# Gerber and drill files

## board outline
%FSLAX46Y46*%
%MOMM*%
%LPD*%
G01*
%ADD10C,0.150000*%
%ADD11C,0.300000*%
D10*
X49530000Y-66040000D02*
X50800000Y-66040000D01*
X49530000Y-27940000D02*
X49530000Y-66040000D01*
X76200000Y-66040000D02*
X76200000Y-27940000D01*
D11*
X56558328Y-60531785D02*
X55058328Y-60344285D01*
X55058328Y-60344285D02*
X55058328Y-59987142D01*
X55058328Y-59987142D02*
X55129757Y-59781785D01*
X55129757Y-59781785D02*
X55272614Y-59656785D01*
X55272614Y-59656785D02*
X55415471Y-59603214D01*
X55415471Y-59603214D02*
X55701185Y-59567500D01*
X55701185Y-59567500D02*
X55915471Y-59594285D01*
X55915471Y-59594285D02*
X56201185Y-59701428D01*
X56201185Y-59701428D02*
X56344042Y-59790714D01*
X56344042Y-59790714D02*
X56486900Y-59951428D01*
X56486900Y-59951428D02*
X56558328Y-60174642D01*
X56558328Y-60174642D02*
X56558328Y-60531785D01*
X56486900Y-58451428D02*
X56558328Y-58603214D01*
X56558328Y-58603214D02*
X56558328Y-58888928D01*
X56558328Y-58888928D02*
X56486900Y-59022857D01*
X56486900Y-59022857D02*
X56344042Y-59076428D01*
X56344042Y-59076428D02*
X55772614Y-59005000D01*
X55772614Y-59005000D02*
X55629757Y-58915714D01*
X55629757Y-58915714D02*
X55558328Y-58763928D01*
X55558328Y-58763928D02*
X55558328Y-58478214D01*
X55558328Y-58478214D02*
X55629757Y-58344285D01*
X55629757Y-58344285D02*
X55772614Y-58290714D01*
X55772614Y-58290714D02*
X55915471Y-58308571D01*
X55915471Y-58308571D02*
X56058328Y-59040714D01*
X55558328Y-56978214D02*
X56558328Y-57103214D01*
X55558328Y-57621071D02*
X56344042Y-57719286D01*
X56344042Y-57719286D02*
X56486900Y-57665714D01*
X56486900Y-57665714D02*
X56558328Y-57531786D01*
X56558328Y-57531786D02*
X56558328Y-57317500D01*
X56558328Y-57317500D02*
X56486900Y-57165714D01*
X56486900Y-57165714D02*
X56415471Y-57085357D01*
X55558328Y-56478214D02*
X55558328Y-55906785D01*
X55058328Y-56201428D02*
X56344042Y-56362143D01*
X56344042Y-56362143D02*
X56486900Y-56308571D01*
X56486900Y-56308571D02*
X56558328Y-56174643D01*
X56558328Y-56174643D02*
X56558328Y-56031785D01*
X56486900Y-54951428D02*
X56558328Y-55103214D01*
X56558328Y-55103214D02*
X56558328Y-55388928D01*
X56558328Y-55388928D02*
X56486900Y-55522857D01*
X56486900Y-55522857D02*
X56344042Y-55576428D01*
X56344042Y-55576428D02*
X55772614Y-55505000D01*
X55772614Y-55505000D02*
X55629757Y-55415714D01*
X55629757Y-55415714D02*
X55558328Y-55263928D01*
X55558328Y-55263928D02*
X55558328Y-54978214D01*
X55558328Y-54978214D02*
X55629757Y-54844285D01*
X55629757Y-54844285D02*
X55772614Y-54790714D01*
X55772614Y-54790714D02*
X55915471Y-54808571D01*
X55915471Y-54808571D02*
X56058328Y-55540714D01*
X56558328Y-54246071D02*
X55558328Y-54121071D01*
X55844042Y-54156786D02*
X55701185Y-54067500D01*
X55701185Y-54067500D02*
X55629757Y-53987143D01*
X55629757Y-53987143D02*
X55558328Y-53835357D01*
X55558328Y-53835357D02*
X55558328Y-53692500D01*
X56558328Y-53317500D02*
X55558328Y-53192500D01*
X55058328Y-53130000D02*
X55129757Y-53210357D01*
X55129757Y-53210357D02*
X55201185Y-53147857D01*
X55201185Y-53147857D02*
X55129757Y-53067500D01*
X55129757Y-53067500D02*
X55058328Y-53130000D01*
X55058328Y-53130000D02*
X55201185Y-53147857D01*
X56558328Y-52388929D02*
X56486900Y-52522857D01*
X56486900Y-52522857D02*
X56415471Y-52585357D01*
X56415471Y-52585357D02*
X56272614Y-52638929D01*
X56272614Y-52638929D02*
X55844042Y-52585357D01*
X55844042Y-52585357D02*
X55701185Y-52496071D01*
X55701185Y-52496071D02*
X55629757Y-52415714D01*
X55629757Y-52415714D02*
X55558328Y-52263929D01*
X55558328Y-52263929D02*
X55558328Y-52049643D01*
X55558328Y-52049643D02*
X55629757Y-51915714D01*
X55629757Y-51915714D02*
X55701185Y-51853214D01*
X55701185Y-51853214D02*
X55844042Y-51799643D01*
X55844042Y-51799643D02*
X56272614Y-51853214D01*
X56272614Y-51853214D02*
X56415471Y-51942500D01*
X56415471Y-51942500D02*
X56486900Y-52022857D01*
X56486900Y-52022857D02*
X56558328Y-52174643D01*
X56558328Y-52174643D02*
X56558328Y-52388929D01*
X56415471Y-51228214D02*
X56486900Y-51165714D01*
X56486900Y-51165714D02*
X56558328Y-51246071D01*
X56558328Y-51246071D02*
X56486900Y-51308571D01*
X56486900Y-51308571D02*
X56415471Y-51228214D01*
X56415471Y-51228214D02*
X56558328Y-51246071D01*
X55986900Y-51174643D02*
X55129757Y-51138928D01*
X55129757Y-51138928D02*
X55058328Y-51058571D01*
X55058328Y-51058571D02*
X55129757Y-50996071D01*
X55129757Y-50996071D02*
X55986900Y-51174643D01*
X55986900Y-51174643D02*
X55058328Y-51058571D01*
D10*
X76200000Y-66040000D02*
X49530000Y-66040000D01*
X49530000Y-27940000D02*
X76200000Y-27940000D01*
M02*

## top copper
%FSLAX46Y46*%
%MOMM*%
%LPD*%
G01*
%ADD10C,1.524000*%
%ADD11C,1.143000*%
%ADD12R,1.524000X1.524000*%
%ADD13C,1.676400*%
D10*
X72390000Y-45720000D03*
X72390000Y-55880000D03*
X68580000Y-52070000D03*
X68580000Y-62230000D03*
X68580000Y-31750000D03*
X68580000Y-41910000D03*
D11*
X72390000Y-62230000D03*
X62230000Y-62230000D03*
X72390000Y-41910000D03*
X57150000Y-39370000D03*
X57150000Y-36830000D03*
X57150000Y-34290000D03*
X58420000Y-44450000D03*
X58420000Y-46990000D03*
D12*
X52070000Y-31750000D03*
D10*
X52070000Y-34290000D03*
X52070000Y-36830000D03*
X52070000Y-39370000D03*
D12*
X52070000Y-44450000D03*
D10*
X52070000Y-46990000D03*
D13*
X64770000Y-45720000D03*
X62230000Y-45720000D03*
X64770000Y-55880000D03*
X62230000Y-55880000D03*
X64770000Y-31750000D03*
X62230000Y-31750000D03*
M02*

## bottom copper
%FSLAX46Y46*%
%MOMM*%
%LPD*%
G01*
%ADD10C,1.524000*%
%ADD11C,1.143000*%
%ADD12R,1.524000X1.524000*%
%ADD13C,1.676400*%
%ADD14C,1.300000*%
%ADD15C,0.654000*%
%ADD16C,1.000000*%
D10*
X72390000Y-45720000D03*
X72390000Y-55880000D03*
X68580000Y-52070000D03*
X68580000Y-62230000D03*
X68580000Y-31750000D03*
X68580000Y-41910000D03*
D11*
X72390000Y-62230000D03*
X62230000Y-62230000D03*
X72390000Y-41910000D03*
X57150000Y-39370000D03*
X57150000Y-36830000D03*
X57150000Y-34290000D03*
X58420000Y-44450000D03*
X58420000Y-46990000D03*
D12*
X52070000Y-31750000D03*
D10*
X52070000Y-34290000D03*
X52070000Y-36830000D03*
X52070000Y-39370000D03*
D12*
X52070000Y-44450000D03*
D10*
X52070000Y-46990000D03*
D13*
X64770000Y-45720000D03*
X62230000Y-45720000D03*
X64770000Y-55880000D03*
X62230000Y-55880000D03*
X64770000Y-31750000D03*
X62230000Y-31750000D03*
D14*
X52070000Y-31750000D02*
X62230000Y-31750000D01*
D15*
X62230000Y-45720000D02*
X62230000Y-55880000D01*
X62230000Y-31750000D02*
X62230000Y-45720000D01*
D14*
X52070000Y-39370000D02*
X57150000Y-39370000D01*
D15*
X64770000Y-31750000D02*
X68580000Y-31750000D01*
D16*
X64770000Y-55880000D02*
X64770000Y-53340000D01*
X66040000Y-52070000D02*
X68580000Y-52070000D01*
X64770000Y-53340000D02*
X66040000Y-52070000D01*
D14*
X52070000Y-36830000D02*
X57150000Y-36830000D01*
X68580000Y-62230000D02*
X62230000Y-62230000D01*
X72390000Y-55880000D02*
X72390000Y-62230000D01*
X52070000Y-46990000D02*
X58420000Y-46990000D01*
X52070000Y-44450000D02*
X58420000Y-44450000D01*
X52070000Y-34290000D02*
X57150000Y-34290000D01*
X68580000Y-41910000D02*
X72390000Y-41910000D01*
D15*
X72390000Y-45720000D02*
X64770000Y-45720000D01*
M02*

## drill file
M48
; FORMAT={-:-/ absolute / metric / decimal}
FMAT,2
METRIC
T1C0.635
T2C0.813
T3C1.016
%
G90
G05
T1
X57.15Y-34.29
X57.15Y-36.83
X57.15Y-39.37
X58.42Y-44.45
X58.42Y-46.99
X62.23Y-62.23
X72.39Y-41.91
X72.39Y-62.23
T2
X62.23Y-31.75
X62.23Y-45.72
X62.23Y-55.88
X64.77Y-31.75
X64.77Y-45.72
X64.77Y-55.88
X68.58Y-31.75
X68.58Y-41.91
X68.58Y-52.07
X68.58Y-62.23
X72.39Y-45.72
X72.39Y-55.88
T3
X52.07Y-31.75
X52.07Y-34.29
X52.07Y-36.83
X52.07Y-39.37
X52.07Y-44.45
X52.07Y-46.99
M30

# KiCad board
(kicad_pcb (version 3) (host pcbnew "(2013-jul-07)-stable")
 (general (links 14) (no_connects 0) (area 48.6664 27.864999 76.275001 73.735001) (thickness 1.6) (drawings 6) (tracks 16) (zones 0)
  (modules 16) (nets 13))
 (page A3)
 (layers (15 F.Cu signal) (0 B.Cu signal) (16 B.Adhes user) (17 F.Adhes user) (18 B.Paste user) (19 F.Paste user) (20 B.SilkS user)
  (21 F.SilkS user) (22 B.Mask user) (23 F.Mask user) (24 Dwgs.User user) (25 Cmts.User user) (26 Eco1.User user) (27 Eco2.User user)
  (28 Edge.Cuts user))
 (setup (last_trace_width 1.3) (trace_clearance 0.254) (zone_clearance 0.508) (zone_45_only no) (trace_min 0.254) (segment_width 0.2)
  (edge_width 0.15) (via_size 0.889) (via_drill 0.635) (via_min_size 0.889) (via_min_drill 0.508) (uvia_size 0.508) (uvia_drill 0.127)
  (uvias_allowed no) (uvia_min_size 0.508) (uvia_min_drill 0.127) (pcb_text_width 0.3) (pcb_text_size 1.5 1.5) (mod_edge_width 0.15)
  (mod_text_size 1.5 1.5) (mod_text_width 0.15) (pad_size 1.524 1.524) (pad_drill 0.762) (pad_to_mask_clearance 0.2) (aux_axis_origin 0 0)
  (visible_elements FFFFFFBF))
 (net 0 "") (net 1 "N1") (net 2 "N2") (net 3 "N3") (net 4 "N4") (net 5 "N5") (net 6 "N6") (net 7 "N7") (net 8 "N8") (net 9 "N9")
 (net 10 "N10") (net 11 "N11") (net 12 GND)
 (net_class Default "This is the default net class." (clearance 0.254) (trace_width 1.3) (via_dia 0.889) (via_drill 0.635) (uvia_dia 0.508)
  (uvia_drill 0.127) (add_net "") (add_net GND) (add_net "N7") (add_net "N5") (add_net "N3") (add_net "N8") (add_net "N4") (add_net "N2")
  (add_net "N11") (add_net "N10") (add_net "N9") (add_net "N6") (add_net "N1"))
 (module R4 (layer F.Cu) (at 72.39 50.8 270) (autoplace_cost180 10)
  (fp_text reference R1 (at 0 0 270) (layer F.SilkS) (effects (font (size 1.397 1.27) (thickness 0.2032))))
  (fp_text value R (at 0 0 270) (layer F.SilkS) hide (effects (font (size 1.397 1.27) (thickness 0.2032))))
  (pad 1 thru_hole circle (at -5.08 0 270) (size 1.524 1.524) (drill 0.8128) (layers *.Cu *.Mask F.SilkS) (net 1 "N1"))
  (pad 2 thru_hole circle (at 5.08 0 270) (size 1.524 1.524) (drill 0.8128) (layers *.Cu *.Mask F.SilkS) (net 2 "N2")))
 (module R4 (layer F.Cu) (at 68.58 57.15 270) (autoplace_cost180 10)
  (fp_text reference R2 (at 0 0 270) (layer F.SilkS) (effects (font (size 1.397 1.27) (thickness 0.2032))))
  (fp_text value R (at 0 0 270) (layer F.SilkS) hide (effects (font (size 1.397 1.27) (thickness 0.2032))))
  (pad 1 thru_hole circle (at -5.08 0 270) (size 1.524 1.524) (drill 0.8128) (layers *.Cu *.Mask F.SilkS) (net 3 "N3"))
  (pad 2 thru_hole circle (at 5.08 0 270) (size 1.524 1.524) (drill 0.8128) (layers *.Cu *.Mask F.SilkS) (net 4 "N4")))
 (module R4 (layer F.Cu) (at 68.58 36.83 270) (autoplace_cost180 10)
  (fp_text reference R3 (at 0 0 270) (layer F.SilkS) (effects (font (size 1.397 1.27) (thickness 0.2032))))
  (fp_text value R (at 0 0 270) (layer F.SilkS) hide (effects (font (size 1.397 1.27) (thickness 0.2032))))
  (pad 1 thru_hole circle (at -5.08 0 270) (size 1.524 1.524) (drill 0.8128) (layers *.Cu *.Mask F.SilkS) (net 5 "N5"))
  (pad 2 thru_hole circle (at 5.08 0 270) (size 1.524 1.524) (drill 0.8128) (layers *.Cu *.Mask F.SilkS) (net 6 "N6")))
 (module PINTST (layer F.Cu) (at 72.39 62.23)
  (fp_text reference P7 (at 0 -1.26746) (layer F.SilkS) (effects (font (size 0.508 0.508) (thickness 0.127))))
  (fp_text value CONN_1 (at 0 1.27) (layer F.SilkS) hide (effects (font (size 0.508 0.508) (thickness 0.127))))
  (pad 1 thru_hole circle (at 0 0) (size 1.143 1.143) (drill 0.635) (layers *.Cu *.Mask F.SilkS) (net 2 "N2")))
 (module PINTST (layer F.Cu) (at 62.23 62.23)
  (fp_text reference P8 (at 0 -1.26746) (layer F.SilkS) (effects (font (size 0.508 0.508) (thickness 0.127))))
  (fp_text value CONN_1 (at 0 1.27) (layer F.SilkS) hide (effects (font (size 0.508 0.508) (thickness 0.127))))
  (pad 1 thru_hole circle (at 0 0) (size 1.143 1.143) (drill 0.635) (layers *.Cu *.Mask F.SilkS) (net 4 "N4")))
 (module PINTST (layer F.Cu) (at 72.39 41.91)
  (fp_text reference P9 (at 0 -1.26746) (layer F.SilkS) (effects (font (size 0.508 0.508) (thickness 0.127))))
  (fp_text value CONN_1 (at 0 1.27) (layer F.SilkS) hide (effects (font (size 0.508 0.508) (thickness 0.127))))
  (pad 1 thru_hole circle (at 0 0) (size 1.143 1.143) (drill 0.635) (layers *.Cu *.Mask F.SilkS) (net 6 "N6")))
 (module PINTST (layer F.Cu) (at 57.15 39.37)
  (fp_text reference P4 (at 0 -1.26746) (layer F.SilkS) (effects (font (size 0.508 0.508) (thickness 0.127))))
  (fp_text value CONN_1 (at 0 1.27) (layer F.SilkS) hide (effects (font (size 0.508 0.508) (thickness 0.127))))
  (pad 1 thru_hole circle (at 0 0) (size 1.143 1.143) (drill 0.635) (layers *.Cu *.Mask F.SilkS) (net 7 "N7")))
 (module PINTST (layer F.Cu) (at 57.15 36.83)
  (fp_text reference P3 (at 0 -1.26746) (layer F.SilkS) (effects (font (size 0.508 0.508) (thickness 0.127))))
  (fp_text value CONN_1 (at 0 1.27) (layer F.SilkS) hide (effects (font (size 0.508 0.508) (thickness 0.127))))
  (pad 1 thru_hole circle (at 0 0) (size 1.143 1.143) (drill 0.635) (layers *.Cu *.Mask F.SilkS) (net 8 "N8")))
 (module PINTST (layer F.Cu) (at 57.15 34.29)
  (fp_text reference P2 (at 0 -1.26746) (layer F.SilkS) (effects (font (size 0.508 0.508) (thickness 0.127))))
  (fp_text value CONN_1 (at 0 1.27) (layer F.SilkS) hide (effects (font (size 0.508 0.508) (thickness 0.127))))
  (pad 1 thru_hole circle (at 0 0) (size 1.143 1.143) (drill 0.635) (layers *.Cu *.Mask F.SilkS) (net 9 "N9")))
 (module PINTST (layer F.Cu) (at 58.42 44.45)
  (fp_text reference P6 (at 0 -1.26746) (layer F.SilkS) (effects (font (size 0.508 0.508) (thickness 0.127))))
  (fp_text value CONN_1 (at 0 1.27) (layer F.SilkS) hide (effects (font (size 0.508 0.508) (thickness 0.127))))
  (pad 1 thru_hole circle (at 0 0) (size 1.143 1.143) (drill 0.635) (layers *.Cu *.Mask F.SilkS) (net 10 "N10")))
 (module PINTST (layer F.Cu) (at 58.42 46.99)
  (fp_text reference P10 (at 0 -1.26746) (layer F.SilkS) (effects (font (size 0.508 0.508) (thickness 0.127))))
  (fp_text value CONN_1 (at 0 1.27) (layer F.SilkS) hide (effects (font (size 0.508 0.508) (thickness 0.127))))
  (pad 1 thru_hole circle (at 0 0) (size 1.143 1.143) (drill 0.635) (layers *.Cu *.Mask F.SilkS) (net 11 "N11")))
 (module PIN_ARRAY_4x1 (layer F.Cu) (at 52.07 35.56 270)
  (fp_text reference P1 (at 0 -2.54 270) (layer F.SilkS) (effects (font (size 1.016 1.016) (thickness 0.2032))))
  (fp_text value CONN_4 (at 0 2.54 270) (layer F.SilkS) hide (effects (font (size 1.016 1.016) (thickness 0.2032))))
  (pad 1 thru_hole rect (at -3.81 0 270) (size 1.524 1.524) (drill 1.016) (layers *.Cu *.Mask F.SilkS) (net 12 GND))
  (pad 2 thru_hole circle (at -1.27 0 270) (size 1.524 1.524) (drill 1.016) (layers *.Cu *.Mask F.SilkS) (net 9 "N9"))
  (pad 3 thru_hole circle (at 1.27 0 270) (size 1.524 1.524) (drill 1.016) (layers *.Cu *.Mask F.SilkS) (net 8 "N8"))
  (pad 4 thru_hole circle (at 3.81 0 270) (size 1.524 1.524) (drill 1.016) (layers *.Cu *.Mask F.SilkS) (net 7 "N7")))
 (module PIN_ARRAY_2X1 (layer F.Cu) (at 52.07 45.72 270)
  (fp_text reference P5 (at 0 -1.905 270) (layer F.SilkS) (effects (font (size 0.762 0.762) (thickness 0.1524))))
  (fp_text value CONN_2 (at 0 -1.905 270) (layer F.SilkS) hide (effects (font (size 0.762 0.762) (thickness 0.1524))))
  (pad 1 thru_hole rect (at -1.27 0 270) (size 1.524 1.524) (drill 1.016) (layers *.Cu *.Mask F.SilkS) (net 10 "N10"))
  (pad 2 thru_hole circle (at 1.27 0 270) (size 1.524 1.524) (drill 1.016) (layers *.Cu *.Mask F.SilkS) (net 11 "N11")))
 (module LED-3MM (layer F.Cu) (at 63.5 45.72 180)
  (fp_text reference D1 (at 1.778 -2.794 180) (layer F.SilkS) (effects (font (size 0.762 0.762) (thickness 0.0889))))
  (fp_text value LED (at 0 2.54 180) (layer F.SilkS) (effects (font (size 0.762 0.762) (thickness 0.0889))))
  (pad 1 thru_hole circle (at -1.27 0 180) (size 1.6764 1.6764) (drill 0.8128) (layers *.Cu *.Mask F.SilkS) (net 1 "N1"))
  (pad 2 thru_hole circle (at 1.27 0 180) (size 1.6764 1.6764) (drill 0.8128) (layers *.Cu *.Mask F.SilkS) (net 12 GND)))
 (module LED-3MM (layer F.Cu) (at 63.5 55.88 180)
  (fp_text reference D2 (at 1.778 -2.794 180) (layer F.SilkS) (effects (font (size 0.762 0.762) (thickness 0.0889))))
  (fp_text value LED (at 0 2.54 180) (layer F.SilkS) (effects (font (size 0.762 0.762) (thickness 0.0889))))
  (pad 1 thru_hole circle (at -1.27 0 180) (size 1.6764 1.6764) (drill 0.8128) (layers *.Cu *.Mask F.SilkS) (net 3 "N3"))
  (pad 2 thru_hole circle (at 1.27 0 180) (size 1.6764 1.6764) (drill 0.8128) (layers *.Cu *.Mask F.SilkS) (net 12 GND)))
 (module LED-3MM (layer F.Cu) (at 63.5 31.75 180)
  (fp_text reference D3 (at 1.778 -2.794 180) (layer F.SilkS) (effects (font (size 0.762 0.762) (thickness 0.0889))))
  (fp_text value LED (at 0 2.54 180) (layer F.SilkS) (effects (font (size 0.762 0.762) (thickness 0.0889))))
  (pad 1 thru_hole circle (at -1.27 0 180) (size 1.6764 1.6764) (drill 0.8128) (layers *.Cu *.Mask F.SilkS) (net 5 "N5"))
  (pad 2 thru_hole circle (at 1.27 0 180) (size 1.6764 1.6764) (drill 0.8128) (layers *.Cu *.Mask F.SilkS) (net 12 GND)))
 (gr_line (start 49.53 66.04) (end 50.8 66.04) (angle 90) (layer Edge.Cuts) (width 0.15))
 (gr_line (start 49.53 27.94) (end 49.53 66.04) (angle 90) (layer Edge.Cuts) (width 0.15))
 (gr_line (start 76.2 66.04) (end 76.2 27.94) (angle 90) (layer Edge.Cuts) (width 0.15))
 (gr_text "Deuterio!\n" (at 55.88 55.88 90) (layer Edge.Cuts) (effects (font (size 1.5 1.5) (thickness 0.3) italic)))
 (gr_line (start 76.2 66.04) (end 49.53 66.04) (angle 90) (layer Edge.Cuts) (width 0.15))
 (gr_line (start 49.53 27.94) (end 76.2 27.94) (angle 90) (layer Edge.Cuts) (width 0.15))
 (segment (start 52.07 31.75) (end 62.23 31.75) (width 1.3) (layer B.Cu) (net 12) (status C00000))
 (segment (start 62.23 45.72) (end 62.23 55.88) (width 0.654) (layer B.Cu) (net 12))
 (segment (start 62.23 31.75) (end 62.23 45.72) (width 0.654) (layer B.Cu) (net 12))
 (segment (start 52.07 39.37) (end 57.15 39.37) (width 1.3) (layer B.Cu) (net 7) (status C00000))
 (segment (start 64.77 31.75) (end 68.58 31.75) (width 0.654) (layer B.Cu) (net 5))
 (segment (start 64.77 55.88) (end 64.77 53.34) (width 1) (layer B.Cu) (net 3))
 (segment (start 66.04 52.07) (end 68.58 52.07) (width 1) (layer B.Cu) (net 3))
 (segment (start 64.77 53.34) (end 66.04 52.07) (width 1) (layer B.Cu) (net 3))
 (segment (start 52.07 36.83) (end 57.15 36.83) (width 1.3) (layer B.Cu) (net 8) (status C00000))
 (segment (start 68.58 62.23) (end 62.23 62.23) (width 1.3) (layer B.Cu) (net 4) (status C00000))
 (segment (start 72.39 55.88) (end 72.39 62.23) (width 1.3) (layer B.Cu) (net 2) (status C00000))
 (segment (start 52.07 46.99) (end 58.42 46.99) (width 1.3) (layer B.Cu) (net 11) (status C00000))
 (segment (start 52.07 44.45) (end 58.42 44.45) (width 1.3) (layer B.Cu) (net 10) (status C00000))
 (segment (start 52.07 34.29) (end 57.15 34.29) (width 1.3) (layer B.Cu) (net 9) (status C00000))
 (segment (start 68.58 41.91) (end 72.39 41.91) (width 1.3) (layer B.Cu) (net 6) (status C00000))
 (segment (start 72.39 45.72) (end 64.77 45.72) (width 0.654) (layer B.Cu) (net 1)))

